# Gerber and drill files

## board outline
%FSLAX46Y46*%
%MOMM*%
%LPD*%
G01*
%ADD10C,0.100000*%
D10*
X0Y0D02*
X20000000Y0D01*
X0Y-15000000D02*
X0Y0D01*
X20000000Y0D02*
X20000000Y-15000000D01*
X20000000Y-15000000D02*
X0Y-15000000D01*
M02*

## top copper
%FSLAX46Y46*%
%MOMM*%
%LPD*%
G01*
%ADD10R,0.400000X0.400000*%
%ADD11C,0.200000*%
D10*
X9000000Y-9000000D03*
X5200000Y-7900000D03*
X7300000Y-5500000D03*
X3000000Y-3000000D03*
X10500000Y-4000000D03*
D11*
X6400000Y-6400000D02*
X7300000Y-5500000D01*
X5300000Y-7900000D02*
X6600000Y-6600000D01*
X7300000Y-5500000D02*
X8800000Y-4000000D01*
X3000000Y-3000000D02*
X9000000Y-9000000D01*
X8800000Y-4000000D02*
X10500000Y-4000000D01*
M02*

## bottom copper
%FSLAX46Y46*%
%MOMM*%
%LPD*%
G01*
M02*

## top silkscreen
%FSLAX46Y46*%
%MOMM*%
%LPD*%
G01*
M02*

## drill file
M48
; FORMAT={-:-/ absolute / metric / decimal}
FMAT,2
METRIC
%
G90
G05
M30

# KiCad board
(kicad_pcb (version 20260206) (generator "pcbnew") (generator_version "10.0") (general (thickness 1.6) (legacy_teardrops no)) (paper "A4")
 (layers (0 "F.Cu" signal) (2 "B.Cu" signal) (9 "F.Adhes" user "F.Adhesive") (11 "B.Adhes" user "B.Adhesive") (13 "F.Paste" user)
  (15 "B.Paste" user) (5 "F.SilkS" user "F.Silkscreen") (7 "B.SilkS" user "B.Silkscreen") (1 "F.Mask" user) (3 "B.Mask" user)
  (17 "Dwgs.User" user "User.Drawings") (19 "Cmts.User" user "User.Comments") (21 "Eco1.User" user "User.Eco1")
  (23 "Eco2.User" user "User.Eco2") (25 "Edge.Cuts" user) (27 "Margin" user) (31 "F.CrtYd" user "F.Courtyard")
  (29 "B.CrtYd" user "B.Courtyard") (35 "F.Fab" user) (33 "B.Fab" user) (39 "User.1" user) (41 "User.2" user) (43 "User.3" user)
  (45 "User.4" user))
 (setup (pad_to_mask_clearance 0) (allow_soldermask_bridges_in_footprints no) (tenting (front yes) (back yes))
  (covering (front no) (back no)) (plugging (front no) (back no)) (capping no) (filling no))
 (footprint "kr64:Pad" (layer "F.Cu") (at 9 9)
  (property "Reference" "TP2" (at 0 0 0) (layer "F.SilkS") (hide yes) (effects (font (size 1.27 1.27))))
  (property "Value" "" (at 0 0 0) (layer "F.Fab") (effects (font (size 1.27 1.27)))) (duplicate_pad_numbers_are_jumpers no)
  (pad "1" smd rect (at 0 0) (size 0.4 0.4) (layers "F.Cu" "F.Mask" "F.Paste") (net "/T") (thermal_bridge_angle 45)))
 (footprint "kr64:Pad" (layer "F.Cu") (at 5.2 7.9)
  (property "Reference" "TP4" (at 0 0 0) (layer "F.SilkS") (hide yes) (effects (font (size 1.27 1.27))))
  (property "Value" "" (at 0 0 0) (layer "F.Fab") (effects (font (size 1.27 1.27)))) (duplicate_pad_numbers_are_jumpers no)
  (pad "1" smd rect (at 0 0) (size 0.4 0.4) (layers "F.Cu" "F.Mask" "F.Paste") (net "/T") (thermal_bridge_angle 45)))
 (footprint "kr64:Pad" (layer "F.Cu") (at 7.3 5.5)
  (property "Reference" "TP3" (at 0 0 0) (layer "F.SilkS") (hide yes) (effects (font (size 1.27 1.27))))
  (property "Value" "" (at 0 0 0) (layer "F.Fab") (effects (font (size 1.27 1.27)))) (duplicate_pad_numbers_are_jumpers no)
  (pad "1" smd rect (at 0 0) (size 0.4 0.4) (layers "F.Cu" "F.Mask" "F.Paste") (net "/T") (thermal_bridge_angle 45)))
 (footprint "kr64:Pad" (layer "F.Cu") (at 3 3)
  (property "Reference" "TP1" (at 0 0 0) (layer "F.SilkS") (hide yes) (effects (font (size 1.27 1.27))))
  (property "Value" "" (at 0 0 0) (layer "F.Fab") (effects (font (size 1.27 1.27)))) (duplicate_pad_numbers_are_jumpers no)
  (pad "1" smd rect (at 0 0) (size 0.4 0.4) (layers "F.Cu" "F.Mask" "F.Paste") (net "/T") (thermal_bridge_angle 45)))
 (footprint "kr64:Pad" (layer "F.Cu") (at 10.5 4)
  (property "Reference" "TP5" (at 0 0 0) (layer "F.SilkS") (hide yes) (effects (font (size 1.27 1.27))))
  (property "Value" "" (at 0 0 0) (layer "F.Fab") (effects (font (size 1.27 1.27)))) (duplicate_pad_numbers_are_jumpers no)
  (pad "1" smd rect (at 0 0) (size 0.4 0.4) (layers "F.Cu" "F.Mask" "F.Paste") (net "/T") (thermal_bridge_angle 45)))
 (gr_line (start 0 0) (end 20 0) (stroke (width 0.1) (type default)) (layer "Edge.Cuts"))
 (gr_line (start 0 15) (end 0 0) (stroke (width 0.1) (type default)) (layer "Edge.Cuts"))
 (gr_line (start 20 0) (end 20 15) (stroke (width 0.1) (type default)) (layer "Edge.Cuts"))
 (gr_line (start 20 15) (end 0 15) (stroke (width 0.1) (type default)) (layer "Edge.Cuts"))
 (segment (start 6.4 6.4) (end 7.3 5.5) (width 0.2) (layer "F.Cu") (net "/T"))
 (segment (start 5.3 7.9) (end 6.6 6.6) (width 0.2) (layer "F.Cu") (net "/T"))
 (segment (start 7.3 5.5) (end 8.8 4) (width 0.2) (layer "F.Cu") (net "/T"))
 (segment (start 3 3) (end 9 9) (width 0.2) (layer "F.Cu") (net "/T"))
 (segment (start 8.8 4) (end 10.5 4) (width 0.2) (layer "F.Cu") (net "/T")))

